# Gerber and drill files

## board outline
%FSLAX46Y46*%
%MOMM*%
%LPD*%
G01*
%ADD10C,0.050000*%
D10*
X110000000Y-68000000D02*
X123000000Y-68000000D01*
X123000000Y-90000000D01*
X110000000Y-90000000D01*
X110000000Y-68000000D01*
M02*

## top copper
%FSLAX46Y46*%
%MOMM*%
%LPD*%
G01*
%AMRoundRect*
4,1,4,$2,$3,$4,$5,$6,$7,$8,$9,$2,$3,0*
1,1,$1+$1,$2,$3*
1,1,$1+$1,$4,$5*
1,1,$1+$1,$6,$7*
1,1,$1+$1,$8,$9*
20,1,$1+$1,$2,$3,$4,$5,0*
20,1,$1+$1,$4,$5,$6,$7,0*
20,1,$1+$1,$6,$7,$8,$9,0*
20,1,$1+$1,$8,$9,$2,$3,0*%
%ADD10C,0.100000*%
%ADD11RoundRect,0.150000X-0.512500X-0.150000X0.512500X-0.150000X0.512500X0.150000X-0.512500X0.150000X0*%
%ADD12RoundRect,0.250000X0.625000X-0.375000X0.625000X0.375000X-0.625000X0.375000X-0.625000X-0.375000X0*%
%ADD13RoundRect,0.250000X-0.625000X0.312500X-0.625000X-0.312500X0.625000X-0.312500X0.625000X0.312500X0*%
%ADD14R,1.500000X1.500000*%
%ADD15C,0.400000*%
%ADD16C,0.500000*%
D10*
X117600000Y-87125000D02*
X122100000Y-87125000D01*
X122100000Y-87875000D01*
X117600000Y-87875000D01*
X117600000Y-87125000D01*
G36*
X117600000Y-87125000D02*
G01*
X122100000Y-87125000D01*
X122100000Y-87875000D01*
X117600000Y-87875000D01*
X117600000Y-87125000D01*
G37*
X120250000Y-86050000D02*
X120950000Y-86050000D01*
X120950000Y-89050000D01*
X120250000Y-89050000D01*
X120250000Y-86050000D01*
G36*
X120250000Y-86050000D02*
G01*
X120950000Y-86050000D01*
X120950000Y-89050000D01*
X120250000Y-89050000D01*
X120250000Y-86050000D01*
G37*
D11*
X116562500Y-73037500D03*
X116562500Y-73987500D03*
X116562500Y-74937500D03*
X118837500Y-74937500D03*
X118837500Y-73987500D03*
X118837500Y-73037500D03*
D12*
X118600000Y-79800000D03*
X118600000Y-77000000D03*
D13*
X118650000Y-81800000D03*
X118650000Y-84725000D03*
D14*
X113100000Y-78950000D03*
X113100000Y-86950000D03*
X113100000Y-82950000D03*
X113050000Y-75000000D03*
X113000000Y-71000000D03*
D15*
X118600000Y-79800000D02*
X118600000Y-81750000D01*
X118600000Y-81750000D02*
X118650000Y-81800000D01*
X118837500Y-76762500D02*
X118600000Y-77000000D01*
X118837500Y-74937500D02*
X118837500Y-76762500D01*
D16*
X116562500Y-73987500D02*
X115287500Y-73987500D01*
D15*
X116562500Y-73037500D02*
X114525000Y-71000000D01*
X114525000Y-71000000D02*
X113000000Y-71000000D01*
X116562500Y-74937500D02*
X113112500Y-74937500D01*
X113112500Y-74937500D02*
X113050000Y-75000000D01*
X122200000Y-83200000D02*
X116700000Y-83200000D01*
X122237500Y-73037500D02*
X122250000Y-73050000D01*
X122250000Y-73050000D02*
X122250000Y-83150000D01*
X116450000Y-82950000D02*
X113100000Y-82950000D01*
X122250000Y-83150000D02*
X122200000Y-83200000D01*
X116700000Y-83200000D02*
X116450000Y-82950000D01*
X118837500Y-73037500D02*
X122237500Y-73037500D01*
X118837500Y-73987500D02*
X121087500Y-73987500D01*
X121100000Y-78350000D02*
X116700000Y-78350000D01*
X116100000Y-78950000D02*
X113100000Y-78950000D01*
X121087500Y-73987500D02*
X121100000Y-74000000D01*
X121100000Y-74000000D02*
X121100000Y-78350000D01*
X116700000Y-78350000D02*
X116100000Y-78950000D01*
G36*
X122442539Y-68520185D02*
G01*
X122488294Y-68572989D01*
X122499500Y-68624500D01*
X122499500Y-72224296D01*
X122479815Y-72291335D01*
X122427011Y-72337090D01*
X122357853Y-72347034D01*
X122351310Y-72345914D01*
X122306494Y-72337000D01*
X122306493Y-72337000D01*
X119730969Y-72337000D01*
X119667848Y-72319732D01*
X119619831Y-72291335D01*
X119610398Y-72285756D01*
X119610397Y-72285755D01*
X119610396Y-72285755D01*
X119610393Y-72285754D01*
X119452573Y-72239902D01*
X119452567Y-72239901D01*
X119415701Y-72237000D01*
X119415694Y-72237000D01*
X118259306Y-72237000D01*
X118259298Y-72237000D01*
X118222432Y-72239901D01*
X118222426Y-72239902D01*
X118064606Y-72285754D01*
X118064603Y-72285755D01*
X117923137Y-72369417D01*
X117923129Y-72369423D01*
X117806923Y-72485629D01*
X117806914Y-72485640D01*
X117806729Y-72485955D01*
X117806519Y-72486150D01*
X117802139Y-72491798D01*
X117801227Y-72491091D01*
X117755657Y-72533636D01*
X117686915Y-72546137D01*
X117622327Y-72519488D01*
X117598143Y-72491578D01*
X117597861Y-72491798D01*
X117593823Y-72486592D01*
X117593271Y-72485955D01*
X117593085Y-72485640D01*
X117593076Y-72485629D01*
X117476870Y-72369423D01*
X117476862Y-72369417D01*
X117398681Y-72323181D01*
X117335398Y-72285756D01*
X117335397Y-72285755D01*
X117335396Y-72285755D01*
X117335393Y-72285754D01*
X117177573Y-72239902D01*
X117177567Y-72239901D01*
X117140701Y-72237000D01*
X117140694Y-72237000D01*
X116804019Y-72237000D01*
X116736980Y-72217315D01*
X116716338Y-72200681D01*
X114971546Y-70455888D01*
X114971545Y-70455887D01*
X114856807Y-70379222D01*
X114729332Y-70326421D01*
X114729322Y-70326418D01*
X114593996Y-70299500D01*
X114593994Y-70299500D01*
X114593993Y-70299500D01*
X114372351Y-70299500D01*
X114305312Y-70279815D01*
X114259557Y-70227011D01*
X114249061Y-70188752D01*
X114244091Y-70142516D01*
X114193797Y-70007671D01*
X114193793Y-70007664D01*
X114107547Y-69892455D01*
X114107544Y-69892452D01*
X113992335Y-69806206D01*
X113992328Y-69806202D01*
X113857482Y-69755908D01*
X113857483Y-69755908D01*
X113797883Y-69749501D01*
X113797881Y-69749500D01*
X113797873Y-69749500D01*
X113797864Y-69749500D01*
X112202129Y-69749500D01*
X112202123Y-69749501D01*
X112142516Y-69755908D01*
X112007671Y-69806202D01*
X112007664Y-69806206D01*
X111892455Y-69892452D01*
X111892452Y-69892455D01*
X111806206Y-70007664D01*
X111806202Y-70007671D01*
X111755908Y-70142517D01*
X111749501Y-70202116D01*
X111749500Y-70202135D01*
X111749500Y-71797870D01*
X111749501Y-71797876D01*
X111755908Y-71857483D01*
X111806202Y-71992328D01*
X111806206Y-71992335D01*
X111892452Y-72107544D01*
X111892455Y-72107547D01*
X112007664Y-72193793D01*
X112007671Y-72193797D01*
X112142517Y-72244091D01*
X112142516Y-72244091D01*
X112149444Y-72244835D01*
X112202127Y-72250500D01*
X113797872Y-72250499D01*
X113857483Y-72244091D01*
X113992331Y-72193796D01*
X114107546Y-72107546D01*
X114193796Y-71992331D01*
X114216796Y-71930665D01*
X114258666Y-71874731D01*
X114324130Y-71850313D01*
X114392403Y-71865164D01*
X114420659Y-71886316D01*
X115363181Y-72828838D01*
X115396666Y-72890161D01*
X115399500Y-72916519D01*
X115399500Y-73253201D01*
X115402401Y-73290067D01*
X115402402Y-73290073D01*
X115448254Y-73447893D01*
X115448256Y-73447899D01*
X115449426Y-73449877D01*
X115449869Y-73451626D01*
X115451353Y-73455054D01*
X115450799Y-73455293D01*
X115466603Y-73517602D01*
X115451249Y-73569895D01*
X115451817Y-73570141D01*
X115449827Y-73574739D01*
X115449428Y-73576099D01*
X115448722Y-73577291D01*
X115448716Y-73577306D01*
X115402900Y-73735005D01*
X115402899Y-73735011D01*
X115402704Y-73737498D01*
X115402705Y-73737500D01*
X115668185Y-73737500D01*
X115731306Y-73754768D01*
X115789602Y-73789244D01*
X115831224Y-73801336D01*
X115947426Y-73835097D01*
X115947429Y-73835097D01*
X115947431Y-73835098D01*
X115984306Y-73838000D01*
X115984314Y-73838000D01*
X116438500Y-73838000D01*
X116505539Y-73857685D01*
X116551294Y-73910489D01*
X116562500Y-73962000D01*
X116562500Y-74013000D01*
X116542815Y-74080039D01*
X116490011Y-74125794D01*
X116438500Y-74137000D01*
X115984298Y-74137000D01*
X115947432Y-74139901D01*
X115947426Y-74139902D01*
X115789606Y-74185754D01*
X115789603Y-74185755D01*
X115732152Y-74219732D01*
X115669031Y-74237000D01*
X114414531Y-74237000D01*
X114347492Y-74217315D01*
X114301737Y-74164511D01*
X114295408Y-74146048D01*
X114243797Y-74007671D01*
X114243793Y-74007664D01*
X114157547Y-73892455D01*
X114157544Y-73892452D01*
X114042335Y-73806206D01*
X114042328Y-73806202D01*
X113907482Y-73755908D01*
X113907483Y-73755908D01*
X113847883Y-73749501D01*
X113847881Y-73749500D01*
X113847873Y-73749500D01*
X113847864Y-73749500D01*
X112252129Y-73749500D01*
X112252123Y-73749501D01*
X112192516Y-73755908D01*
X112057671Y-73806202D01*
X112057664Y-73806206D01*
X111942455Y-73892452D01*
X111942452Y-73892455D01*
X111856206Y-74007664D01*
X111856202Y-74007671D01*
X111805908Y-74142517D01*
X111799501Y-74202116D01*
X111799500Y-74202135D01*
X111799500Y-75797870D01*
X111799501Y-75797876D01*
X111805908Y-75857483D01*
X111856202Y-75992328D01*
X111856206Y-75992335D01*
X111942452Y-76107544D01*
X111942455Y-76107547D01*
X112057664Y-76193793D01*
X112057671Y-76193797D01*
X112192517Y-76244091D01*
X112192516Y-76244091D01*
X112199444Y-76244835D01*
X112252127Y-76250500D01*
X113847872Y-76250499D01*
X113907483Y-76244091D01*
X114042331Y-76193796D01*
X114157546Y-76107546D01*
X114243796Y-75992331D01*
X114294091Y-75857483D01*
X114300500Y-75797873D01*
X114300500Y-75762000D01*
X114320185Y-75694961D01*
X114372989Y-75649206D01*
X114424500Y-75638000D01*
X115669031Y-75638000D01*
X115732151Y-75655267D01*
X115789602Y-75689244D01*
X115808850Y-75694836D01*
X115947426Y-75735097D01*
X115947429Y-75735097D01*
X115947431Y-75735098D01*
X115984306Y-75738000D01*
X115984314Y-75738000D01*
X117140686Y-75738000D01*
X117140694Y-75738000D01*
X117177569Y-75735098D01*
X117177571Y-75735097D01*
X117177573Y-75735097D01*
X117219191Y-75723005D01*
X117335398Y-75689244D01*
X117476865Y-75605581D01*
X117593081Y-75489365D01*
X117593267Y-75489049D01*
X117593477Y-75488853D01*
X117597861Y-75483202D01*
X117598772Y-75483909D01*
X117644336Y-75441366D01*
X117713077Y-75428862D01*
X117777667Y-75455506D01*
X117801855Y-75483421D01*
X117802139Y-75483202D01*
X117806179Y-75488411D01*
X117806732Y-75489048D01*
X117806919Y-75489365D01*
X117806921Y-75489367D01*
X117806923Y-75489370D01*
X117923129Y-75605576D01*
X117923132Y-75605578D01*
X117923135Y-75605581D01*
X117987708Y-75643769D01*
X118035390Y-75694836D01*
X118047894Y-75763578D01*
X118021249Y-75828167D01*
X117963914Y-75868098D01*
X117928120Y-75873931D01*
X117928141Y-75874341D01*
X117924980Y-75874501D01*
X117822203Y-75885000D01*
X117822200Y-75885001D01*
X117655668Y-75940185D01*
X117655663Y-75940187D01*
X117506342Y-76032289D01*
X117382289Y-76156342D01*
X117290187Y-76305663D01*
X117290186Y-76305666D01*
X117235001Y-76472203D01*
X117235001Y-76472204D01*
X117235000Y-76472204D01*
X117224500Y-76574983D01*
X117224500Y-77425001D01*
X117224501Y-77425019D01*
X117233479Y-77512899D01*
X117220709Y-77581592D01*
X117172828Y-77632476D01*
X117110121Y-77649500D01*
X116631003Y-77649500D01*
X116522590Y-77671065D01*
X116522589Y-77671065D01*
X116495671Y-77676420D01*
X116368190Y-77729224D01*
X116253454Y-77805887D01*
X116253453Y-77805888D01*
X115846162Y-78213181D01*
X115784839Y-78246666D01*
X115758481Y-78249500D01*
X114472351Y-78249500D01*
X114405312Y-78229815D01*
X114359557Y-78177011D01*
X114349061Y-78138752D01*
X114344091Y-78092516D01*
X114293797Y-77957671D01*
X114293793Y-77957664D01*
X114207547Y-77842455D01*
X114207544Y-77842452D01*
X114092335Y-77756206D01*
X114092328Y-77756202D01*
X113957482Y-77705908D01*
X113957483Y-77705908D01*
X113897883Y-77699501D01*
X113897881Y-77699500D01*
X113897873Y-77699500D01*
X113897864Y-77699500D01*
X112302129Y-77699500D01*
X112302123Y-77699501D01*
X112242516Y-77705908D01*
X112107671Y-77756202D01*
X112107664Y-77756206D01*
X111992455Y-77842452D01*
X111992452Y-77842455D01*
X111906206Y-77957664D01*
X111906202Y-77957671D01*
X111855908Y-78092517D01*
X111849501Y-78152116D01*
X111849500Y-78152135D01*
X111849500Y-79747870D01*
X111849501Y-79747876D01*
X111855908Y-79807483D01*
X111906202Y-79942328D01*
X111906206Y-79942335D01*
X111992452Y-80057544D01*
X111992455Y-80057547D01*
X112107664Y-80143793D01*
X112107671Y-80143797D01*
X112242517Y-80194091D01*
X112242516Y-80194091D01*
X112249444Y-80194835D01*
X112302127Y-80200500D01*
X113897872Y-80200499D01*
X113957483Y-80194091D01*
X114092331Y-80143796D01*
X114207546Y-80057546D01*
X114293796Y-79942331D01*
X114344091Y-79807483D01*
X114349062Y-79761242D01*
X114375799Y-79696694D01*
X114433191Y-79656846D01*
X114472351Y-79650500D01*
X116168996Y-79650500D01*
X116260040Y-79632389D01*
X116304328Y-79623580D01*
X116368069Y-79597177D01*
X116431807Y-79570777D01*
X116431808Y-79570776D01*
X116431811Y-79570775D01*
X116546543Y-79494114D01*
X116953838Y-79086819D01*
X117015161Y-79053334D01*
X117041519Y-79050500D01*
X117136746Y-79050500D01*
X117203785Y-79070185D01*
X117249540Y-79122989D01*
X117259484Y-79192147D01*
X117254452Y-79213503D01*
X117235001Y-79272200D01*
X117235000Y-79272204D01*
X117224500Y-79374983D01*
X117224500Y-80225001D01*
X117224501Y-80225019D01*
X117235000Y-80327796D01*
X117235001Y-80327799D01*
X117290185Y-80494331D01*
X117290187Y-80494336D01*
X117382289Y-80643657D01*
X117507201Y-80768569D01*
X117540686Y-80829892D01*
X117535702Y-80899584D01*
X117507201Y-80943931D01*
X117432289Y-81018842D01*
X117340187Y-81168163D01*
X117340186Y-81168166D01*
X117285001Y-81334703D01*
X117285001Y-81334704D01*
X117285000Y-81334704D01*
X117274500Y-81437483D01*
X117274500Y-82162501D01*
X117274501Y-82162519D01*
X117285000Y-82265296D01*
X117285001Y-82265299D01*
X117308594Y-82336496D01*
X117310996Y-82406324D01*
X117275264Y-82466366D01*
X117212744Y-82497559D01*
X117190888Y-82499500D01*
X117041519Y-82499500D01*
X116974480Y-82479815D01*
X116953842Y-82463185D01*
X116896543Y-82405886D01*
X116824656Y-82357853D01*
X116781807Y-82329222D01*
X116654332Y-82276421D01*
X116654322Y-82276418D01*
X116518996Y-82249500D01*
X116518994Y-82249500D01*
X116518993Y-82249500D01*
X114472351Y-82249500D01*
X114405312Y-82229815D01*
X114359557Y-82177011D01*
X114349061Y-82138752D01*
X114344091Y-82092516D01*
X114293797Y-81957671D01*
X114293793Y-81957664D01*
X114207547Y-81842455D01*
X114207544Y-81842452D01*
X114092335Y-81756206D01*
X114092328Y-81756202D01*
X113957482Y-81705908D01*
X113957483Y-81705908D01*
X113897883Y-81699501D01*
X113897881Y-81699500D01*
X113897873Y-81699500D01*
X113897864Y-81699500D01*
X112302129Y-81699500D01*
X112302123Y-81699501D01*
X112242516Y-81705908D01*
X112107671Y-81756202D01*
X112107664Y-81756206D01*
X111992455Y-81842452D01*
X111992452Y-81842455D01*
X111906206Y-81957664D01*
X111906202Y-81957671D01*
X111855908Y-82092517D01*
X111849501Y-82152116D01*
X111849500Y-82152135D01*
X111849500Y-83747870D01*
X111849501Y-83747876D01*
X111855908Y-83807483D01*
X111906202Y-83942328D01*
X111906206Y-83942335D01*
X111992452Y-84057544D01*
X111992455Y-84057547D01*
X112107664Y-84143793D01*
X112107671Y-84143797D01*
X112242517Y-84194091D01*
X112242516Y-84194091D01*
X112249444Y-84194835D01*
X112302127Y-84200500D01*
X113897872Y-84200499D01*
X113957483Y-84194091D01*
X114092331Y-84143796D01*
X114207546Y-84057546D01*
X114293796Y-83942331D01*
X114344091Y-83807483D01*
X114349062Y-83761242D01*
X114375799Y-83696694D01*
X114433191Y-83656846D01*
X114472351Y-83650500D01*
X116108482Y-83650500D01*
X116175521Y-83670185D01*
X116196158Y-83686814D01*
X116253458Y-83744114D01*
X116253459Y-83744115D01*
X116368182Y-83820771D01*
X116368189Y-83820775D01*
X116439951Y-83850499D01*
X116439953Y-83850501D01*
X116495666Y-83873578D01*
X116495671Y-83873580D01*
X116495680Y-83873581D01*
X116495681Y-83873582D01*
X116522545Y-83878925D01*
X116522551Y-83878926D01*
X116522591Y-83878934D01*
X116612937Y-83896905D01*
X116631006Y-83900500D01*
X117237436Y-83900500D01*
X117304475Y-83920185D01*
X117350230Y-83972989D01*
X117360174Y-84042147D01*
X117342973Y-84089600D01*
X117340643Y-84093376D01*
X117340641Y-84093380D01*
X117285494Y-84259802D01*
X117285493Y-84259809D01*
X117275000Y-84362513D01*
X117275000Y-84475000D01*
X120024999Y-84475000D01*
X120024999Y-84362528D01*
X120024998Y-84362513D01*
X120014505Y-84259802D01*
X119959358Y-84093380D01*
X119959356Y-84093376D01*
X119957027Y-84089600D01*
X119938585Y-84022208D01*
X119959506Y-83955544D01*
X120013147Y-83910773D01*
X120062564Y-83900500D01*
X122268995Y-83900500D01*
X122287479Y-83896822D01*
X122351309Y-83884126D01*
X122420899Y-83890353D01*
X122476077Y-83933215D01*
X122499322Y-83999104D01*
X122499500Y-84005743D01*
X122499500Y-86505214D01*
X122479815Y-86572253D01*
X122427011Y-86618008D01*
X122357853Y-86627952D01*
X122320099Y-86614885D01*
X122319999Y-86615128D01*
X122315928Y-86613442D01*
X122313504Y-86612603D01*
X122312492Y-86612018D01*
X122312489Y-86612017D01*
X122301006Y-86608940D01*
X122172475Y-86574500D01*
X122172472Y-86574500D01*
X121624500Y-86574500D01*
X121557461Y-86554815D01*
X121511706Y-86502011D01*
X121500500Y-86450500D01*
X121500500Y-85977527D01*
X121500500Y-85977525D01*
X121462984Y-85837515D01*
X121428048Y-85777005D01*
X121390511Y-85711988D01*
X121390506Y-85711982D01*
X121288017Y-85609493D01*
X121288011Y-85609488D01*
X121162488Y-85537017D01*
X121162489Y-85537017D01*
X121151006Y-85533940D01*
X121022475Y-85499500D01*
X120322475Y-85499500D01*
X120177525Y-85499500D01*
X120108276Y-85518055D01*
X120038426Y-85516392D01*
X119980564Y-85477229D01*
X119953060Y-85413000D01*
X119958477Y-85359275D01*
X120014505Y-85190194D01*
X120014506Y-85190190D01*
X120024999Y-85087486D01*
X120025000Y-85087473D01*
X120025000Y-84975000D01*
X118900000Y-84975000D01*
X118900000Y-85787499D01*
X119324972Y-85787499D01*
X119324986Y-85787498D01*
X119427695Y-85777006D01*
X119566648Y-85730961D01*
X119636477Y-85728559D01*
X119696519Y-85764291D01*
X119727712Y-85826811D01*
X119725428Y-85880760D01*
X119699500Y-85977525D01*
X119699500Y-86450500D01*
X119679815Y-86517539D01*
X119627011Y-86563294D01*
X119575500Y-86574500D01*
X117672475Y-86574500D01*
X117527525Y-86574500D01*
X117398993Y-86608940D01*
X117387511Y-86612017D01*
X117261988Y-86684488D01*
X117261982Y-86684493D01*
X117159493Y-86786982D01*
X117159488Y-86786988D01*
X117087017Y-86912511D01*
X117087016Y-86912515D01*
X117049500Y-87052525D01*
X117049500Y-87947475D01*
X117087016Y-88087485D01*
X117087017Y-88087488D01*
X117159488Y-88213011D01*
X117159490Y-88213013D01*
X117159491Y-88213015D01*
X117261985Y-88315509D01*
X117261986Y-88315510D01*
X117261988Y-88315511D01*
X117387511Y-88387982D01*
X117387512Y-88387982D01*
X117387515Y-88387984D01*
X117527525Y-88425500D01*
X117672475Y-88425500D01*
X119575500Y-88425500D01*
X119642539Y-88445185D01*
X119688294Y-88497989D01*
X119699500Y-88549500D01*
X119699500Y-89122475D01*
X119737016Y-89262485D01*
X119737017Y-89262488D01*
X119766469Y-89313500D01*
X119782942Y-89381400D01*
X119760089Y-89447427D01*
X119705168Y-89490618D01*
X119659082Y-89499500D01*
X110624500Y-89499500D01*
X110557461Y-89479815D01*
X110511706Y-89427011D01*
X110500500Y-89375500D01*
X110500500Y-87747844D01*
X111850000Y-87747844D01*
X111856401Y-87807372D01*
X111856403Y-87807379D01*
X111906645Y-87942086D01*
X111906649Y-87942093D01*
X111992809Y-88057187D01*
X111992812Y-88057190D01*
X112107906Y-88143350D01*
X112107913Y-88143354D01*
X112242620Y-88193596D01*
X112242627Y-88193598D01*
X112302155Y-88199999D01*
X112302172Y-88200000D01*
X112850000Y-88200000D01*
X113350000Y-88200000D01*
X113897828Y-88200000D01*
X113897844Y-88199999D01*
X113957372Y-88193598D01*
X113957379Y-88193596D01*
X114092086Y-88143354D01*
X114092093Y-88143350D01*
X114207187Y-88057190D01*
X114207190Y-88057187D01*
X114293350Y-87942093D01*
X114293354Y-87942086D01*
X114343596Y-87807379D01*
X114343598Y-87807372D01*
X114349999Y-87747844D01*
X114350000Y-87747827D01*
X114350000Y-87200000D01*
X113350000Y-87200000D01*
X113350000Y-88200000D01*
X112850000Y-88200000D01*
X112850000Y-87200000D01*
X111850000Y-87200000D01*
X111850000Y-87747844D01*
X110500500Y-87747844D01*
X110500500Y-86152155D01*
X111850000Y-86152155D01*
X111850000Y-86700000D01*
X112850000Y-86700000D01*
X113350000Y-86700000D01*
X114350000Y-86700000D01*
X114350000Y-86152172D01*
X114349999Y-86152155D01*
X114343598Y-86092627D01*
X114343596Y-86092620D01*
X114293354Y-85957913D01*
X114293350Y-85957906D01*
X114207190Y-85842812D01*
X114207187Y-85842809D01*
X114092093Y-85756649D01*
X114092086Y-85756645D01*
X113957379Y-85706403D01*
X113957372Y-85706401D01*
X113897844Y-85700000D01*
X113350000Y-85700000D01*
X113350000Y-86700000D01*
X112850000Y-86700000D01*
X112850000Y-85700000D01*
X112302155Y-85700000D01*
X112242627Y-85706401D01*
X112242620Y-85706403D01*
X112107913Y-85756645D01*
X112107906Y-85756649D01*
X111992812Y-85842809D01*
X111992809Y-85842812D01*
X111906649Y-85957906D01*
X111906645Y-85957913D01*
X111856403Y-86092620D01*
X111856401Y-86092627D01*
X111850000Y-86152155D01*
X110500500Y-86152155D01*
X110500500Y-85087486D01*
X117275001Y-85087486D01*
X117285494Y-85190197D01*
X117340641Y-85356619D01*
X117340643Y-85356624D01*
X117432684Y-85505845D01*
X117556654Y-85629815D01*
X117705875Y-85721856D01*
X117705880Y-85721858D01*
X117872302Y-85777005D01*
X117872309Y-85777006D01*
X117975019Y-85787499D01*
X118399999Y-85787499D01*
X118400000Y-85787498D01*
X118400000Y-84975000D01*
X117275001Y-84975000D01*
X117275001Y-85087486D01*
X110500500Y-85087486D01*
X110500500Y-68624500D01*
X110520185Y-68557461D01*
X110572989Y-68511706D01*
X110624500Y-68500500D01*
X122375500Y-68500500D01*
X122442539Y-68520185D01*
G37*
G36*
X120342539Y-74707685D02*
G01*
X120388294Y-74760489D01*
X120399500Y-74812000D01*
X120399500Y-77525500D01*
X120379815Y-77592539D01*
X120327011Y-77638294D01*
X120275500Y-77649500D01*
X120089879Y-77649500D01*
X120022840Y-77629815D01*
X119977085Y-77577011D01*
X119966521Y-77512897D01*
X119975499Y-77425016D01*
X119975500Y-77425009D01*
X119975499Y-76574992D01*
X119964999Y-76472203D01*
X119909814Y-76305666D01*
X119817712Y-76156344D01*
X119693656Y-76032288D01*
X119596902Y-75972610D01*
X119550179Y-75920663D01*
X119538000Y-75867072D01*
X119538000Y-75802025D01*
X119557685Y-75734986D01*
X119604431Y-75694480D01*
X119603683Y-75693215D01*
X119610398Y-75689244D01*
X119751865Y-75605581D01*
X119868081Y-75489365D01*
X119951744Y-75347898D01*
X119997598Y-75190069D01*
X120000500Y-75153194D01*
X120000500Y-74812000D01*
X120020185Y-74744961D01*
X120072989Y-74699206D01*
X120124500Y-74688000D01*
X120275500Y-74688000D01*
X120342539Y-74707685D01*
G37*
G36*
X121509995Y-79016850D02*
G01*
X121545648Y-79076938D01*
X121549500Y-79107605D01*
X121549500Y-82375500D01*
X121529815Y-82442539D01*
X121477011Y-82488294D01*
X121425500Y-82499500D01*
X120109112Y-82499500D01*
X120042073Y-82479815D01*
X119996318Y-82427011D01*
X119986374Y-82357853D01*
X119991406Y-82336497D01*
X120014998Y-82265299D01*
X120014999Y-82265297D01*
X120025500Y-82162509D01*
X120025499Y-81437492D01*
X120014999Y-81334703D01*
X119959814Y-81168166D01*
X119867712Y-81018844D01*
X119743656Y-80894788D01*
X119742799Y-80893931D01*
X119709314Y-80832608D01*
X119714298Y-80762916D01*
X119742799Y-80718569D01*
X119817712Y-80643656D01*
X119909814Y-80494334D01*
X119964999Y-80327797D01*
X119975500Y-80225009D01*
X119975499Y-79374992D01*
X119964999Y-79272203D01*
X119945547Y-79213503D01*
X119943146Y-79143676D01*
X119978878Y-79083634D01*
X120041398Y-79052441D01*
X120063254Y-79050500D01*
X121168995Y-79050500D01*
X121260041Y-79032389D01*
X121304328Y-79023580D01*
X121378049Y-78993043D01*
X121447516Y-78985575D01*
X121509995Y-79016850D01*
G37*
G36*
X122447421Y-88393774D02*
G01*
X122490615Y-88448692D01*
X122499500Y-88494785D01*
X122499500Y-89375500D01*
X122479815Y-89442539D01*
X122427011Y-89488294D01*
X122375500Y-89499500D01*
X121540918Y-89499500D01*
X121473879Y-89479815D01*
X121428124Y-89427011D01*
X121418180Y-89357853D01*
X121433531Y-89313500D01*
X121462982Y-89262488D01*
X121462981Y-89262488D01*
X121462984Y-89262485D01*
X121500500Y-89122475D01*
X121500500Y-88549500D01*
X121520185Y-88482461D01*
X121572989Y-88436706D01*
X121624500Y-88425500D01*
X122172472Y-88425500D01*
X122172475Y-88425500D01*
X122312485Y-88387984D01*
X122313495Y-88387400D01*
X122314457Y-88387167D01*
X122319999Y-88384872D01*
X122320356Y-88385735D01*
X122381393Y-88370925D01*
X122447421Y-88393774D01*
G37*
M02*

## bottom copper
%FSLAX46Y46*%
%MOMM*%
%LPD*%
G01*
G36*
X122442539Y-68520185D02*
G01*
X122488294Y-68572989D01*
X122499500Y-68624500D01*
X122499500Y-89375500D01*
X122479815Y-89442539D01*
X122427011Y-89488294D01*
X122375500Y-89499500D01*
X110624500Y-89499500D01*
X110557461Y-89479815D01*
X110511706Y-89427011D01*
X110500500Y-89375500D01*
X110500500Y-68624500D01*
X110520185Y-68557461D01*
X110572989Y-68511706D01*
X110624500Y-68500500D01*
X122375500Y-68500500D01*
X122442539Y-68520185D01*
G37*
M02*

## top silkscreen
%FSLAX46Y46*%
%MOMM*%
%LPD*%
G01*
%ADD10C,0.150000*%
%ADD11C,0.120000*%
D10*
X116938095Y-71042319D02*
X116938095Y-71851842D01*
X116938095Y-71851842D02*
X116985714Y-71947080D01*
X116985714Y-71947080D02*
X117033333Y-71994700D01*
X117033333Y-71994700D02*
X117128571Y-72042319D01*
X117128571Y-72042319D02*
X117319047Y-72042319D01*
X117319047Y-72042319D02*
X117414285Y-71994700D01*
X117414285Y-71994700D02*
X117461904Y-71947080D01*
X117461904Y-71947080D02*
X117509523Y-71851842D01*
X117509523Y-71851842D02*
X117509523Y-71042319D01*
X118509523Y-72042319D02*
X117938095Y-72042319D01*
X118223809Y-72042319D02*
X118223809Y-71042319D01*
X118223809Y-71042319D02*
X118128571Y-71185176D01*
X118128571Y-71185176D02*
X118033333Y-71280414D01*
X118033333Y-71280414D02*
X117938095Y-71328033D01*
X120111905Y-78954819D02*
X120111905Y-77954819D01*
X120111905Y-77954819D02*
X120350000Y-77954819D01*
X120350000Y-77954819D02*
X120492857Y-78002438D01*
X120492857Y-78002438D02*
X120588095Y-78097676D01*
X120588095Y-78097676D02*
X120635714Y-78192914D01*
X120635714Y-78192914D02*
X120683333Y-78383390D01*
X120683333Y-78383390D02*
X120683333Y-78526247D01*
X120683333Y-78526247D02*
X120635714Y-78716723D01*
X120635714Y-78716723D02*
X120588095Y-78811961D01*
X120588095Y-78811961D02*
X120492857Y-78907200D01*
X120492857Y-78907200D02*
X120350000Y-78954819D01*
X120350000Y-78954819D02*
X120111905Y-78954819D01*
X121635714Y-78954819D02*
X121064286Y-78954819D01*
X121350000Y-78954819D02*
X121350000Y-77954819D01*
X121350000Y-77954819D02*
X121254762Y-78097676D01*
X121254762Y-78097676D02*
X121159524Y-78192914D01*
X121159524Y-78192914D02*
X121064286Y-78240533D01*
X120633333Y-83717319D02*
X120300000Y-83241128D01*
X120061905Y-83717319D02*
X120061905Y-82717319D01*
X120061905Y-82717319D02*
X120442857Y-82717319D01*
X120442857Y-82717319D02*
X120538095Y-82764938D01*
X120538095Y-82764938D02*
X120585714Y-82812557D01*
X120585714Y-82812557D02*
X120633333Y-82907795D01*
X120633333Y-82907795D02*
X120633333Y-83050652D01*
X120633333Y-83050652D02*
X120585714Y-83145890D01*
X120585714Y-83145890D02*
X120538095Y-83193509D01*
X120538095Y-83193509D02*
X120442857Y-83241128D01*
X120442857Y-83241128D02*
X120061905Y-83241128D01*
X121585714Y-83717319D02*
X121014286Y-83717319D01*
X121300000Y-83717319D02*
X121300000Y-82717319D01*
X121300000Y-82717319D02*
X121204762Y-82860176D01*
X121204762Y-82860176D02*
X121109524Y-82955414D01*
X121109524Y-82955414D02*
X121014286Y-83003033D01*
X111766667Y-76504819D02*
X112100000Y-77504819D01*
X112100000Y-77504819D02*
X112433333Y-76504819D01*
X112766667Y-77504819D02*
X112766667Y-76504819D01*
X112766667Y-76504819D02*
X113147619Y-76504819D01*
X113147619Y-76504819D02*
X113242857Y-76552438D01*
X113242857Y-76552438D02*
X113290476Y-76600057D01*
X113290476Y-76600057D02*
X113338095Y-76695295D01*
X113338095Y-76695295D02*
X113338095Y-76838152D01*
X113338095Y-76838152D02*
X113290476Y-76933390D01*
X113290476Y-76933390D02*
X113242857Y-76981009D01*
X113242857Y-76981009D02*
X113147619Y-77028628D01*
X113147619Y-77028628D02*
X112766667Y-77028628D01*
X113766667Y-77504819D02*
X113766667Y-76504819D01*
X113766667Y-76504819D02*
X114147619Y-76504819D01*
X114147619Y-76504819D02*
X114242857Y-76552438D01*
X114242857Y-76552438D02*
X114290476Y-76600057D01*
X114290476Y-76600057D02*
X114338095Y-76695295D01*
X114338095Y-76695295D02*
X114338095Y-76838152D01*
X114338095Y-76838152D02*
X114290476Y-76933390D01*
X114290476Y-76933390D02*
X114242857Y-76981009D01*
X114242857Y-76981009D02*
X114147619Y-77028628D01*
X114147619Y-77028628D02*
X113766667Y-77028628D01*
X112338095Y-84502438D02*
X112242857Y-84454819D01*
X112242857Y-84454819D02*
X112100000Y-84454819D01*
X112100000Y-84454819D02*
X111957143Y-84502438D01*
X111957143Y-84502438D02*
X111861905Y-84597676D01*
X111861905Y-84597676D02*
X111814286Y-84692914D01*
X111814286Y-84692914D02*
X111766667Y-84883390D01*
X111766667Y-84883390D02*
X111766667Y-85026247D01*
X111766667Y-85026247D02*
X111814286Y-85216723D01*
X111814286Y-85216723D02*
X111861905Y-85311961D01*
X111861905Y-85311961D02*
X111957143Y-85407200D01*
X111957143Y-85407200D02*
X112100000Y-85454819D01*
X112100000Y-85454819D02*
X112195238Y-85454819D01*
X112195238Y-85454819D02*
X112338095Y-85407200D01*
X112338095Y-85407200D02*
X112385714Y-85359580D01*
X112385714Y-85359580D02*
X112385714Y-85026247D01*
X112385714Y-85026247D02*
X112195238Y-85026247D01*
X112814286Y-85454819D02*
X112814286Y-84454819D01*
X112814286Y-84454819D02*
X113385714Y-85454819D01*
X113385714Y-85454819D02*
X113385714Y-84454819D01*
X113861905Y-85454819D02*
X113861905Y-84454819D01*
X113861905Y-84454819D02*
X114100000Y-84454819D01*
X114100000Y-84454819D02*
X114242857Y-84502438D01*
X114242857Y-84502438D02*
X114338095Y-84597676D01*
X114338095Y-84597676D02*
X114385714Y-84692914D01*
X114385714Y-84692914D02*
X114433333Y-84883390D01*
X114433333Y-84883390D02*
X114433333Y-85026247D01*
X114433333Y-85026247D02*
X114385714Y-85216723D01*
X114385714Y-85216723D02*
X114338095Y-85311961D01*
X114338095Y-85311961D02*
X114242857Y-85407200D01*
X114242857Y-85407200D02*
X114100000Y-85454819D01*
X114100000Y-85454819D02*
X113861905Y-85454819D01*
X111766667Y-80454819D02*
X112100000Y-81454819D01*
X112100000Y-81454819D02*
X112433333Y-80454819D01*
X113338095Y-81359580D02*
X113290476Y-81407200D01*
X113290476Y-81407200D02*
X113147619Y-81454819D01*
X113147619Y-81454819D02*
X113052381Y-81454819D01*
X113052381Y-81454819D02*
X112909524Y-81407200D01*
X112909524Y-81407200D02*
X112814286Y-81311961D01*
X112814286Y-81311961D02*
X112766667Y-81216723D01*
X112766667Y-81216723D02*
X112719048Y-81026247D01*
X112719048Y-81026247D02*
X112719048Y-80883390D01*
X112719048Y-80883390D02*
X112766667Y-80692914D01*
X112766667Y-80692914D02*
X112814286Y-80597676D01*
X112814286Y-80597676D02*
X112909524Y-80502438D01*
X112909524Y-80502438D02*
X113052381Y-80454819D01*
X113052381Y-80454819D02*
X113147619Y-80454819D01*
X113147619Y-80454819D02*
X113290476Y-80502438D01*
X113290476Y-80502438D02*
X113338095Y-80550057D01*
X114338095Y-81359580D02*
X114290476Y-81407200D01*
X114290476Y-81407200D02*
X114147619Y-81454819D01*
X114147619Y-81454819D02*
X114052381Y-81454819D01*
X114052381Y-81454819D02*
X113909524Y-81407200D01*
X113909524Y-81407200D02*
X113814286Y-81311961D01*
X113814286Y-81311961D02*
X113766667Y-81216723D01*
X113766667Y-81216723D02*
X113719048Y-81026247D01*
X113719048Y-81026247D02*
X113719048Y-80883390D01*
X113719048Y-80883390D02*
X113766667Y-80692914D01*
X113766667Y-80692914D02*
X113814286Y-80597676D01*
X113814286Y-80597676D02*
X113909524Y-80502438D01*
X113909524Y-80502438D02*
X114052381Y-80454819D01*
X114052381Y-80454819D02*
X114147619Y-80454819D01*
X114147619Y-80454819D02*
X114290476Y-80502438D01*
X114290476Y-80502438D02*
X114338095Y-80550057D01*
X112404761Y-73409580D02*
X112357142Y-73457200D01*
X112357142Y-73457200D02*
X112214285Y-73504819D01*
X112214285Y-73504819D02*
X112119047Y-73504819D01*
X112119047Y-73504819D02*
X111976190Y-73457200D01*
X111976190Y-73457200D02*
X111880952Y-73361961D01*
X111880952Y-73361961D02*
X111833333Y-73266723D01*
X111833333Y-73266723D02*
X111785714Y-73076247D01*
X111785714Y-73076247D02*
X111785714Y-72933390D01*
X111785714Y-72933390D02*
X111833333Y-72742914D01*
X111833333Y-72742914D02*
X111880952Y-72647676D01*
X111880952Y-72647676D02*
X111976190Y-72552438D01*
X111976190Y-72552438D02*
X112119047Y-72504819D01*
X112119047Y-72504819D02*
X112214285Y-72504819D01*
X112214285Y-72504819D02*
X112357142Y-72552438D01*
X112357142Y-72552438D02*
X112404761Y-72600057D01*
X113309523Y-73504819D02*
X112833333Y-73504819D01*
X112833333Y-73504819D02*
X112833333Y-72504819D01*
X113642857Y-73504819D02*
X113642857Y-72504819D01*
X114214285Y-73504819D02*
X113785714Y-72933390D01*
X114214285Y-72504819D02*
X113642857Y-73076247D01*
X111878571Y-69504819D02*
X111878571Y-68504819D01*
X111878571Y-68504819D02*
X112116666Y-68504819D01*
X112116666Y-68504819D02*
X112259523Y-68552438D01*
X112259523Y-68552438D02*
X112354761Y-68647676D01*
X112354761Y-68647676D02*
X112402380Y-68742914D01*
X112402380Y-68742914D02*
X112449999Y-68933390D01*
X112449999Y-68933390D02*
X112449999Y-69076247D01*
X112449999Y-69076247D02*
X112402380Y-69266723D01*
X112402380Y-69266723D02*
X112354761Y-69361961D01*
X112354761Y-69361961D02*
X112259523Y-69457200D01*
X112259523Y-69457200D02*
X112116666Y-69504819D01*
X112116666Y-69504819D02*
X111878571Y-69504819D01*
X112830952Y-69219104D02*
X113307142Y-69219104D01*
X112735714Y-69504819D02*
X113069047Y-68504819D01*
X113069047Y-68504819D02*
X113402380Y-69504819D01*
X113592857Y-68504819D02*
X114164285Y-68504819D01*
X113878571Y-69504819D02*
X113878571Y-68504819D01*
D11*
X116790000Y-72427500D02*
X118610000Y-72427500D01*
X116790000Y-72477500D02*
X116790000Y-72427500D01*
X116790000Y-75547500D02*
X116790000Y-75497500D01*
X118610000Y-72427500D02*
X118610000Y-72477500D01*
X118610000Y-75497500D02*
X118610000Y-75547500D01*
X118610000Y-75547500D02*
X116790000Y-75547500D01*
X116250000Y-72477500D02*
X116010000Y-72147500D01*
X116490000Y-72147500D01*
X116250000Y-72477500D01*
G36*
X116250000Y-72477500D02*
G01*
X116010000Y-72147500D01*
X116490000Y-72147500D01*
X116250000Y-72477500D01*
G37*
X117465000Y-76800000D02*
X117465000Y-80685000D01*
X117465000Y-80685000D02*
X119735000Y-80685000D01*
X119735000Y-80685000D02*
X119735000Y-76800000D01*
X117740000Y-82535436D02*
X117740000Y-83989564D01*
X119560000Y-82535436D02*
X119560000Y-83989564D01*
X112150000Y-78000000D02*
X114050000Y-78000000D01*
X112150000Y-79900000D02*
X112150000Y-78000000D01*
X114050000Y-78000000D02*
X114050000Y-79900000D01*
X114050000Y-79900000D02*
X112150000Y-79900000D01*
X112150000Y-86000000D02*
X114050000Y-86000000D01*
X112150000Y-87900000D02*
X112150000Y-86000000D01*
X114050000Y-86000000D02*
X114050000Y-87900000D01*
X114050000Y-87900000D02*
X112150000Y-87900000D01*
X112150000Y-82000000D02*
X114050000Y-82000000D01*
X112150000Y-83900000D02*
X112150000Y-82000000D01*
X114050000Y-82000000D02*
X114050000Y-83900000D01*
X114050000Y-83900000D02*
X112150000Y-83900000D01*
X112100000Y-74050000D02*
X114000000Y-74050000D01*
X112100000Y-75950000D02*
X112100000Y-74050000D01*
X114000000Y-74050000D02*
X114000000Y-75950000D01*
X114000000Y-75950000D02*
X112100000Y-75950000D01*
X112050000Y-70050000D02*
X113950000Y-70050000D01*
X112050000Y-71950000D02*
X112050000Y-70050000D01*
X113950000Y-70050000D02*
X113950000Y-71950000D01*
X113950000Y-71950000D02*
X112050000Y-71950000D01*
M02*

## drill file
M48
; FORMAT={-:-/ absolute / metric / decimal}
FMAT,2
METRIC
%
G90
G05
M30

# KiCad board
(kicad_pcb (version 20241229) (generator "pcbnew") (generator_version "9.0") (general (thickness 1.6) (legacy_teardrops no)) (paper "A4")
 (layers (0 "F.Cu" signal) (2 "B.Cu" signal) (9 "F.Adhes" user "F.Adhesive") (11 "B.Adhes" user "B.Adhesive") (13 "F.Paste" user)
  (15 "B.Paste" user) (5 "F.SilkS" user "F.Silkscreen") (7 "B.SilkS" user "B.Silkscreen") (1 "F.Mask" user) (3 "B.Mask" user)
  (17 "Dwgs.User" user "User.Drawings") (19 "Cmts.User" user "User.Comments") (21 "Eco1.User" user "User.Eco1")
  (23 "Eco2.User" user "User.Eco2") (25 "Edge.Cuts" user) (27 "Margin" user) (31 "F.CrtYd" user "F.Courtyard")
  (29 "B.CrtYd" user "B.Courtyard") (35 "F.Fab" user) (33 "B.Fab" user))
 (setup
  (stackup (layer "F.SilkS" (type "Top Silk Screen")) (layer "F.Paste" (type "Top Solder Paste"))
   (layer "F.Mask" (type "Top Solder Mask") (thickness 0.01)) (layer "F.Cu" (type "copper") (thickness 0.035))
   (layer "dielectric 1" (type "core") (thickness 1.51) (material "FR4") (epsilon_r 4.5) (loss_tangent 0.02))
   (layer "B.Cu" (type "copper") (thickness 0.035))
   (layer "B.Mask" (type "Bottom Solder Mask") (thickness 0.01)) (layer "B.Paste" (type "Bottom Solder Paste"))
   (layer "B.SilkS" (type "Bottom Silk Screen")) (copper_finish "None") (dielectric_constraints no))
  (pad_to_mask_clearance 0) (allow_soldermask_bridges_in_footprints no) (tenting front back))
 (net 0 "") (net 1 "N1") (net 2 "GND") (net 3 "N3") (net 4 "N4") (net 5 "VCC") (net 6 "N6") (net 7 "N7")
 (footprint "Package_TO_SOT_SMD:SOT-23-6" (layer "F.Cu") (at 117.7 73.9875)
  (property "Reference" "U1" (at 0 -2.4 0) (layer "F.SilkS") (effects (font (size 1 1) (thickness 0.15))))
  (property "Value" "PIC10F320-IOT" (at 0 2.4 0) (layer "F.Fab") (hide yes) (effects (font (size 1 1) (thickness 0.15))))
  (fp_line (start -0.91 -1.56) (end 0.91 -1.56) (stroke (width 0.12) (type solid)) (layer "F.SilkS"))
  (fp_line (start -0.91 -1.51) (end -0.91 -1.56) (stroke (width 0.12) (type solid)) (layer "F.SilkS"))
  (fp_line (start -0.91 1.56) (end -0.91 1.51) (stroke (width 0.12) (type solid)) (layer "F.SilkS"))
  (fp_line (start 0.91 -1.56) (end 0.91 -1.51) (stroke (width 0.12) (type solid)) (layer "F.SilkS"))
  (fp_line (start 0.91 1.51) (end 0.91 1.56) (stroke (width 0.12) (type solid)) (layer "F.SilkS"))
  (fp_line (start 0.91 1.56) (end -0.91 1.56) (stroke (width 0.12) (type solid)) (layer "F.SilkS"))
  (fp_poly (pts (xy -1.45 -1.51) (xy -1.69 -1.84) (xy -1.21 -1.84)) (stroke (width 0.12) (type solid)) (fill yes) (layer "F.SilkS"))
  (pad "1" smd roundrect (at -1.1375 -0.95) (size 1.325 0.6) (layers "F.Cu" "F.Mask" "F.Paste") (roundrect_rratio 0.25) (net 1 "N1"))
  (pad "2" smd roundrect (at -1.1375 0) (size 1.325 0.6) (layers "F.Cu" "F.Mask" "F.Paste") (roundrect_rratio 0.25) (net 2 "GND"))
  (pad "3" smd roundrect (at -1.1375 0.95) (size 1.325 0.6) (layers "F.Cu" "F.Mask" "F.Paste") (roundrect_rratio 0.25) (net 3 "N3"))
  (pad "4" smd roundrect (at 1.1375 0.95) (size 1.325 0.6) (layers "F.Cu" "F.Mask" "F.Paste") (roundrect_rratio 0.25) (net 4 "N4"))
  (pad "5" smd roundrect (at 1.1375 0) (size 1.325 0.6) (layers "F.Cu" "F.Mask" "F.Paste") (roundrect_rratio 0.25) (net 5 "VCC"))
  (pad "6" smd roundrect (at 1.1375 -0.95) (size 1.325 0.6) (layers "F.Cu" "F.Mask" "F.Paste") (roundrect_rratio 0.25) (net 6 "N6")))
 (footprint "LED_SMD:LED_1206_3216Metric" (layer "F.Cu") (at 118.6 78.4 90)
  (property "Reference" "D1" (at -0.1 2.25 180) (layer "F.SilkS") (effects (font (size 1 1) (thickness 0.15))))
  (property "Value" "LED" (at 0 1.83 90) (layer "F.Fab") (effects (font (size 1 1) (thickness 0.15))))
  (fp_line (start 1.6 -1.135) (end -2.285 -1.135) (stroke (width 0.12) (type solid)) (layer "F.SilkS"))
  (fp_line (start -2.285 -1.135) (end -2.285 1.135) (stroke (width 0.12) (type solid)) (layer "F.SilkS"))
  (fp_line (start -2.285 1.135) (end 1.6 1.135) (stroke (width 0.12) (type solid)) (layer "F.SilkS"))
  (pad "1" smd roundrect (at -1.4 0 90) (size 1.25 1.75) (layers "F.Cu" "F.Mask" "F.Paste") (roundrect_rratio 0.2) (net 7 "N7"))
  (pad "2" smd roundrect (at 1.4 0 90) (size 1.25 1.75) (layers "F.Cu" "F.Mask" "F.Paste") (roundrect_rratio 0.2) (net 4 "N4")))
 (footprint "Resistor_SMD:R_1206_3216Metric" (layer "F.Cu") (at 118.65 83.2625 -90)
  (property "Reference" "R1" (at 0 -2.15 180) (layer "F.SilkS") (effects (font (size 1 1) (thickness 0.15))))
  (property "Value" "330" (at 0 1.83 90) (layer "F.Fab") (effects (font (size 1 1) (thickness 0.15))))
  (fp_line (start -0.727064 0.91) (end 0.727064 0.91) (stroke (width 0.12) (type solid)) (layer "F.SilkS"))
  (fp_line (start -0.727064 -0.91) (end 0.727064 -0.91) (stroke (width 0.12) (type solid)) (layer "F.SilkS"))
  (pad "1" smd roundrect (at -1.4625 0 270) (size 1.125 1.75) (layers "F.Cu" "F.Mask" "F.Paste") (roundrect_rratio 0.222222) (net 7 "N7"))
  (pad "2" smd roundrect (at 1.4625 0 270) (size 1.125 1.75) (layers "F.Cu" "F.Mask" "F.Paste") (roundrect_rratio 0.222222) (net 2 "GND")))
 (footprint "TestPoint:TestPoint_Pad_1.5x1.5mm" (layer "F.Cu") (at 113.1 78.95)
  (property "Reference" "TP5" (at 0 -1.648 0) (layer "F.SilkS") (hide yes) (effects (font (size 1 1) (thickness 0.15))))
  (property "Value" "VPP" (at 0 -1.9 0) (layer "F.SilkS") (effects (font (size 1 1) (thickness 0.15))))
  (fp_line (start -0.95 -0.95) (end 0.95 -0.95) (stroke (width 0.12) (type solid)) (layer "F.SilkS"))
  (fp_line (start -0.95 0.95) (end -0.95 -0.95) (stroke (width 0.12) (type solid)) (layer "F.SilkS"))
  (fp_line (start 0.95 -0.95) (end 0.95 0.95) (stroke (width 0.12) (type solid)) (layer "F.SilkS"))
  (fp_line (start 0.95 0.95) (end -0.95 0.95) (stroke (width 0.12) (type solid)) (layer "F.SilkS"))
  (pad "1" smd rect (at 0 0) (size 1.5 1.5) (layers "F.Cu" "F.Mask") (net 5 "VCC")))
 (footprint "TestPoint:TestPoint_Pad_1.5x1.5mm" (layer "F.Cu") (at 113.1 86.95)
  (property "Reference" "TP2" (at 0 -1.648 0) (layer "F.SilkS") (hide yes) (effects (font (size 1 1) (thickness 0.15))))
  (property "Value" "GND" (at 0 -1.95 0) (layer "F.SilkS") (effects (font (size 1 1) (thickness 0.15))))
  (fp_line (start -0.95 -0.95) (end 0.95 -0.95) (stroke (width 0.12) (type solid)) (layer "F.SilkS"))
  (fp_line (start -0.95 0.95) (end -0.95 -0.95) (stroke (width 0.12) (type solid)) (layer "F.SilkS"))
  (fp_line (start 0.95 -0.95) (end 0.95 0.95) (stroke (width 0.12) (type solid)) (layer "F.SilkS"))
  (fp_line (start 0.95 0.95) (end -0.95 0.95) (stroke (width 0.12) (type solid)) (layer "F.SilkS"))
  (pad "1" smd rect (at 0 0) (size 1.5 1.5) (layers "F.Cu" "F.Mask") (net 2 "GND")))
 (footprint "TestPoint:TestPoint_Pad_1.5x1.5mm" (layer "F.Cu") (at 113.1 82.95)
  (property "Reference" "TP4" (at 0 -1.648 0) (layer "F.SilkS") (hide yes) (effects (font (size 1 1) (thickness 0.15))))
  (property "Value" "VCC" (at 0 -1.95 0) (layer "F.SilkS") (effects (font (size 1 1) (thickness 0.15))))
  (fp_line (start -0.95 -0.95) (end 0.95 -0.95) (stroke (width 0.12) (type solid)) (layer "F.SilkS"))
  (fp_line (start -0.95 0.95) (end -0.95 -0.95) (stroke (width 0.12) (type solid)) (layer "F.SilkS"))
  (fp_line (start 0.95 -0.95) (end 0.95 0.95) (stroke (width 0.12) (type solid)) (layer "F.SilkS"))
  (fp_line (start 0.95 0.95) (end -0.95 0.95) (stroke (width 0.12) (type solid)) (layer "F.SilkS"))
  (pad "1" smd rect (at 0 0) (size 1.5 1.5) (layers "F.Cu" "F.Mask") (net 6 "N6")))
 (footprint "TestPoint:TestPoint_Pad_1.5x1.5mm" (layer "F.Cu") (at 113.05 75)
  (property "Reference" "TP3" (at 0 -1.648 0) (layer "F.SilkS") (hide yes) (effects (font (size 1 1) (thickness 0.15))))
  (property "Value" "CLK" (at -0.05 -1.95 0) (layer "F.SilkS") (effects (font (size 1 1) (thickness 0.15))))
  (fp_line (start -0.95 -0.95) (end 0.95 -0.95) (stroke (width 0.12) (type solid)) (layer "F.SilkS"))
  (fp_line (start -0.95 0.95) (end -0.95 -0.95) (stroke (width 0.12) (type solid)) (layer "F.SilkS"))
  (fp_line (start 0.95 -0.95) (end 0.95 0.95) (stroke (width 0.12) (type solid)) (layer "F.SilkS"))
  (fp_line (start 0.95 0.95) (end -0.95 0.95) (stroke (width 0.12) (type solid)) (layer "F.SilkS"))
  (pad "1" smd rect (at 0 0) (size 1.5 1.5) (layers "F.Cu" "F.Mask") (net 3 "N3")))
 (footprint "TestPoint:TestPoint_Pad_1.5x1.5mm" (layer "F.Cu") (at 113 71)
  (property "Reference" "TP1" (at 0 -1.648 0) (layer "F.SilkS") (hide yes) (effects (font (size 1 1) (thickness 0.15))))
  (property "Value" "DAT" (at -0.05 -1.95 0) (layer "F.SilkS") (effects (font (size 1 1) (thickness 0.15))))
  (fp_line (start -0.95 -0.95) (end 0.95 -0.95) (stroke (width 0.12) (type solid)) (layer "F.SilkS"))
  (fp_line (start -0.95 0.95) (end -0.95 -0.95) (stroke (width 0.12) (type solid)) (layer "F.SilkS"))
  (fp_line (start 0.95 -0.95) (end 0.95 0.95) (stroke (width 0.12) (type solid)) (layer "F.SilkS"))
  (fp_line (start 0.95 0.95) (end -0.95 0.95) (stroke (width 0.12) (type solid)) (layer "F.SilkS"))
  (pad "1" smd rect (at 0 0) (size 1.5 1.5) (layers "F.Cu" "F.Mask") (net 1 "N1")))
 (gr_rect (start 122.1 87.125) (end 117.6 87.875) (stroke (width 0.1) (type solid)) (fill yes) (layer "F.Cu"))
 (gr_rect (start 120.95 86.05) (end 120.25 89.05) (stroke (width 0.1) (type solid)) (fill yes) (layer "F.Cu"))
 (gr_rect (start 110 68) (end 123 90) (stroke (width 0.05) (type default)) (fill no) (layer "Edge.Cuts"))
 (segment (start 118.6 79.8) (end 118.6 81.75) (width 0.4) (layer "F.Cu") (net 7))
 (segment (start 118.6 81.75) (end 118.65 81.8) (width 0.4) (layer "F.Cu") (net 7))
 (segment (start 118.8375 76.7625) (end 118.6 77) (width 0.4) (layer "F.Cu") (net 4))
 (segment (start 118.8375 74.9375) (end 118.8375 76.7625) (width 0.4) (layer "F.Cu") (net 4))
 (segment (start 116.5625 73.9875) (end 115.2875 73.9875) (width 0.5) (layer "F.Cu") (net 2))
 (segment (start 116.5625 73.0375) (end 114.525 71) (width 0.4) (layer "F.Cu") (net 1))
 (segment (start 114.525 71) (end 113 71) (width 0.4) (layer "F.Cu") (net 1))
 (segment (start 116.5625 74.9375) (end 113.1125 74.9375) (width 0.4) (layer "F.Cu") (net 3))
 (segment (start 113.1125 74.9375) (end 113.05 75) (width 0.4) (layer "F.Cu") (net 3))
 (segment (start 122.2 83.2) (end 116.7 83.2) (width 0.4) (layer "F.Cu") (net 6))
 (segment (start 122.2375 73.0375) (end 122.25 73.05) (width 0.4) (layer "F.Cu") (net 6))
 (segment (start 122.25 73.05) (end 122.25 83.15) (width 0.4) (layer "F.Cu") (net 6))
 (segment (start 116.45 82.95) (end 113.1 82.95) (width 0.4) (layer "F.Cu") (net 6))
 (segment (start 122.25 83.15) (end 122.2 83.2) (width 0.4) (layer "F.Cu") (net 6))
 (segment (start 116.7 83.2) (end 116.45 82.95) (width 0.4) (layer "F.Cu") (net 6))
 (segment (start 118.8375 73.0375) (end 122.2375 73.0375) (width 0.4) (layer "F.Cu") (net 6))
 (segment (start 118.8375 73.9875) (end 121.0875 73.9875) (width 0.4) (layer "F.Cu") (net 5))
 (segment (start 121.1 78.35) (end 116.7 78.35) (width 0.4) (layer "F.Cu") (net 5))
 (segment (start 116.1 78.95) (end 113.1 78.95) (width 0.4) (layer "F.Cu") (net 5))
 (segment (start 121.0875 73.9875) (end 121.1 74) (width 0.4) (layer "F.Cu") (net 5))
 (segment (start 121.1 74) (end 121.1 78.35) (width 0.4) (layer "F.Cu") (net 5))
 (segment (start 116.7 78.35) (end 116.1 78.95) (width 0.4) (layer "F.Cu") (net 5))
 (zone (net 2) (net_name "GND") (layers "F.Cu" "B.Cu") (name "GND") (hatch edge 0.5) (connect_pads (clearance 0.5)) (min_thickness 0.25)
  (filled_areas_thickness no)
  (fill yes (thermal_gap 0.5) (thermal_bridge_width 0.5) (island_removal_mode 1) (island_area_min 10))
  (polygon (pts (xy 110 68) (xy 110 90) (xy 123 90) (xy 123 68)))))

